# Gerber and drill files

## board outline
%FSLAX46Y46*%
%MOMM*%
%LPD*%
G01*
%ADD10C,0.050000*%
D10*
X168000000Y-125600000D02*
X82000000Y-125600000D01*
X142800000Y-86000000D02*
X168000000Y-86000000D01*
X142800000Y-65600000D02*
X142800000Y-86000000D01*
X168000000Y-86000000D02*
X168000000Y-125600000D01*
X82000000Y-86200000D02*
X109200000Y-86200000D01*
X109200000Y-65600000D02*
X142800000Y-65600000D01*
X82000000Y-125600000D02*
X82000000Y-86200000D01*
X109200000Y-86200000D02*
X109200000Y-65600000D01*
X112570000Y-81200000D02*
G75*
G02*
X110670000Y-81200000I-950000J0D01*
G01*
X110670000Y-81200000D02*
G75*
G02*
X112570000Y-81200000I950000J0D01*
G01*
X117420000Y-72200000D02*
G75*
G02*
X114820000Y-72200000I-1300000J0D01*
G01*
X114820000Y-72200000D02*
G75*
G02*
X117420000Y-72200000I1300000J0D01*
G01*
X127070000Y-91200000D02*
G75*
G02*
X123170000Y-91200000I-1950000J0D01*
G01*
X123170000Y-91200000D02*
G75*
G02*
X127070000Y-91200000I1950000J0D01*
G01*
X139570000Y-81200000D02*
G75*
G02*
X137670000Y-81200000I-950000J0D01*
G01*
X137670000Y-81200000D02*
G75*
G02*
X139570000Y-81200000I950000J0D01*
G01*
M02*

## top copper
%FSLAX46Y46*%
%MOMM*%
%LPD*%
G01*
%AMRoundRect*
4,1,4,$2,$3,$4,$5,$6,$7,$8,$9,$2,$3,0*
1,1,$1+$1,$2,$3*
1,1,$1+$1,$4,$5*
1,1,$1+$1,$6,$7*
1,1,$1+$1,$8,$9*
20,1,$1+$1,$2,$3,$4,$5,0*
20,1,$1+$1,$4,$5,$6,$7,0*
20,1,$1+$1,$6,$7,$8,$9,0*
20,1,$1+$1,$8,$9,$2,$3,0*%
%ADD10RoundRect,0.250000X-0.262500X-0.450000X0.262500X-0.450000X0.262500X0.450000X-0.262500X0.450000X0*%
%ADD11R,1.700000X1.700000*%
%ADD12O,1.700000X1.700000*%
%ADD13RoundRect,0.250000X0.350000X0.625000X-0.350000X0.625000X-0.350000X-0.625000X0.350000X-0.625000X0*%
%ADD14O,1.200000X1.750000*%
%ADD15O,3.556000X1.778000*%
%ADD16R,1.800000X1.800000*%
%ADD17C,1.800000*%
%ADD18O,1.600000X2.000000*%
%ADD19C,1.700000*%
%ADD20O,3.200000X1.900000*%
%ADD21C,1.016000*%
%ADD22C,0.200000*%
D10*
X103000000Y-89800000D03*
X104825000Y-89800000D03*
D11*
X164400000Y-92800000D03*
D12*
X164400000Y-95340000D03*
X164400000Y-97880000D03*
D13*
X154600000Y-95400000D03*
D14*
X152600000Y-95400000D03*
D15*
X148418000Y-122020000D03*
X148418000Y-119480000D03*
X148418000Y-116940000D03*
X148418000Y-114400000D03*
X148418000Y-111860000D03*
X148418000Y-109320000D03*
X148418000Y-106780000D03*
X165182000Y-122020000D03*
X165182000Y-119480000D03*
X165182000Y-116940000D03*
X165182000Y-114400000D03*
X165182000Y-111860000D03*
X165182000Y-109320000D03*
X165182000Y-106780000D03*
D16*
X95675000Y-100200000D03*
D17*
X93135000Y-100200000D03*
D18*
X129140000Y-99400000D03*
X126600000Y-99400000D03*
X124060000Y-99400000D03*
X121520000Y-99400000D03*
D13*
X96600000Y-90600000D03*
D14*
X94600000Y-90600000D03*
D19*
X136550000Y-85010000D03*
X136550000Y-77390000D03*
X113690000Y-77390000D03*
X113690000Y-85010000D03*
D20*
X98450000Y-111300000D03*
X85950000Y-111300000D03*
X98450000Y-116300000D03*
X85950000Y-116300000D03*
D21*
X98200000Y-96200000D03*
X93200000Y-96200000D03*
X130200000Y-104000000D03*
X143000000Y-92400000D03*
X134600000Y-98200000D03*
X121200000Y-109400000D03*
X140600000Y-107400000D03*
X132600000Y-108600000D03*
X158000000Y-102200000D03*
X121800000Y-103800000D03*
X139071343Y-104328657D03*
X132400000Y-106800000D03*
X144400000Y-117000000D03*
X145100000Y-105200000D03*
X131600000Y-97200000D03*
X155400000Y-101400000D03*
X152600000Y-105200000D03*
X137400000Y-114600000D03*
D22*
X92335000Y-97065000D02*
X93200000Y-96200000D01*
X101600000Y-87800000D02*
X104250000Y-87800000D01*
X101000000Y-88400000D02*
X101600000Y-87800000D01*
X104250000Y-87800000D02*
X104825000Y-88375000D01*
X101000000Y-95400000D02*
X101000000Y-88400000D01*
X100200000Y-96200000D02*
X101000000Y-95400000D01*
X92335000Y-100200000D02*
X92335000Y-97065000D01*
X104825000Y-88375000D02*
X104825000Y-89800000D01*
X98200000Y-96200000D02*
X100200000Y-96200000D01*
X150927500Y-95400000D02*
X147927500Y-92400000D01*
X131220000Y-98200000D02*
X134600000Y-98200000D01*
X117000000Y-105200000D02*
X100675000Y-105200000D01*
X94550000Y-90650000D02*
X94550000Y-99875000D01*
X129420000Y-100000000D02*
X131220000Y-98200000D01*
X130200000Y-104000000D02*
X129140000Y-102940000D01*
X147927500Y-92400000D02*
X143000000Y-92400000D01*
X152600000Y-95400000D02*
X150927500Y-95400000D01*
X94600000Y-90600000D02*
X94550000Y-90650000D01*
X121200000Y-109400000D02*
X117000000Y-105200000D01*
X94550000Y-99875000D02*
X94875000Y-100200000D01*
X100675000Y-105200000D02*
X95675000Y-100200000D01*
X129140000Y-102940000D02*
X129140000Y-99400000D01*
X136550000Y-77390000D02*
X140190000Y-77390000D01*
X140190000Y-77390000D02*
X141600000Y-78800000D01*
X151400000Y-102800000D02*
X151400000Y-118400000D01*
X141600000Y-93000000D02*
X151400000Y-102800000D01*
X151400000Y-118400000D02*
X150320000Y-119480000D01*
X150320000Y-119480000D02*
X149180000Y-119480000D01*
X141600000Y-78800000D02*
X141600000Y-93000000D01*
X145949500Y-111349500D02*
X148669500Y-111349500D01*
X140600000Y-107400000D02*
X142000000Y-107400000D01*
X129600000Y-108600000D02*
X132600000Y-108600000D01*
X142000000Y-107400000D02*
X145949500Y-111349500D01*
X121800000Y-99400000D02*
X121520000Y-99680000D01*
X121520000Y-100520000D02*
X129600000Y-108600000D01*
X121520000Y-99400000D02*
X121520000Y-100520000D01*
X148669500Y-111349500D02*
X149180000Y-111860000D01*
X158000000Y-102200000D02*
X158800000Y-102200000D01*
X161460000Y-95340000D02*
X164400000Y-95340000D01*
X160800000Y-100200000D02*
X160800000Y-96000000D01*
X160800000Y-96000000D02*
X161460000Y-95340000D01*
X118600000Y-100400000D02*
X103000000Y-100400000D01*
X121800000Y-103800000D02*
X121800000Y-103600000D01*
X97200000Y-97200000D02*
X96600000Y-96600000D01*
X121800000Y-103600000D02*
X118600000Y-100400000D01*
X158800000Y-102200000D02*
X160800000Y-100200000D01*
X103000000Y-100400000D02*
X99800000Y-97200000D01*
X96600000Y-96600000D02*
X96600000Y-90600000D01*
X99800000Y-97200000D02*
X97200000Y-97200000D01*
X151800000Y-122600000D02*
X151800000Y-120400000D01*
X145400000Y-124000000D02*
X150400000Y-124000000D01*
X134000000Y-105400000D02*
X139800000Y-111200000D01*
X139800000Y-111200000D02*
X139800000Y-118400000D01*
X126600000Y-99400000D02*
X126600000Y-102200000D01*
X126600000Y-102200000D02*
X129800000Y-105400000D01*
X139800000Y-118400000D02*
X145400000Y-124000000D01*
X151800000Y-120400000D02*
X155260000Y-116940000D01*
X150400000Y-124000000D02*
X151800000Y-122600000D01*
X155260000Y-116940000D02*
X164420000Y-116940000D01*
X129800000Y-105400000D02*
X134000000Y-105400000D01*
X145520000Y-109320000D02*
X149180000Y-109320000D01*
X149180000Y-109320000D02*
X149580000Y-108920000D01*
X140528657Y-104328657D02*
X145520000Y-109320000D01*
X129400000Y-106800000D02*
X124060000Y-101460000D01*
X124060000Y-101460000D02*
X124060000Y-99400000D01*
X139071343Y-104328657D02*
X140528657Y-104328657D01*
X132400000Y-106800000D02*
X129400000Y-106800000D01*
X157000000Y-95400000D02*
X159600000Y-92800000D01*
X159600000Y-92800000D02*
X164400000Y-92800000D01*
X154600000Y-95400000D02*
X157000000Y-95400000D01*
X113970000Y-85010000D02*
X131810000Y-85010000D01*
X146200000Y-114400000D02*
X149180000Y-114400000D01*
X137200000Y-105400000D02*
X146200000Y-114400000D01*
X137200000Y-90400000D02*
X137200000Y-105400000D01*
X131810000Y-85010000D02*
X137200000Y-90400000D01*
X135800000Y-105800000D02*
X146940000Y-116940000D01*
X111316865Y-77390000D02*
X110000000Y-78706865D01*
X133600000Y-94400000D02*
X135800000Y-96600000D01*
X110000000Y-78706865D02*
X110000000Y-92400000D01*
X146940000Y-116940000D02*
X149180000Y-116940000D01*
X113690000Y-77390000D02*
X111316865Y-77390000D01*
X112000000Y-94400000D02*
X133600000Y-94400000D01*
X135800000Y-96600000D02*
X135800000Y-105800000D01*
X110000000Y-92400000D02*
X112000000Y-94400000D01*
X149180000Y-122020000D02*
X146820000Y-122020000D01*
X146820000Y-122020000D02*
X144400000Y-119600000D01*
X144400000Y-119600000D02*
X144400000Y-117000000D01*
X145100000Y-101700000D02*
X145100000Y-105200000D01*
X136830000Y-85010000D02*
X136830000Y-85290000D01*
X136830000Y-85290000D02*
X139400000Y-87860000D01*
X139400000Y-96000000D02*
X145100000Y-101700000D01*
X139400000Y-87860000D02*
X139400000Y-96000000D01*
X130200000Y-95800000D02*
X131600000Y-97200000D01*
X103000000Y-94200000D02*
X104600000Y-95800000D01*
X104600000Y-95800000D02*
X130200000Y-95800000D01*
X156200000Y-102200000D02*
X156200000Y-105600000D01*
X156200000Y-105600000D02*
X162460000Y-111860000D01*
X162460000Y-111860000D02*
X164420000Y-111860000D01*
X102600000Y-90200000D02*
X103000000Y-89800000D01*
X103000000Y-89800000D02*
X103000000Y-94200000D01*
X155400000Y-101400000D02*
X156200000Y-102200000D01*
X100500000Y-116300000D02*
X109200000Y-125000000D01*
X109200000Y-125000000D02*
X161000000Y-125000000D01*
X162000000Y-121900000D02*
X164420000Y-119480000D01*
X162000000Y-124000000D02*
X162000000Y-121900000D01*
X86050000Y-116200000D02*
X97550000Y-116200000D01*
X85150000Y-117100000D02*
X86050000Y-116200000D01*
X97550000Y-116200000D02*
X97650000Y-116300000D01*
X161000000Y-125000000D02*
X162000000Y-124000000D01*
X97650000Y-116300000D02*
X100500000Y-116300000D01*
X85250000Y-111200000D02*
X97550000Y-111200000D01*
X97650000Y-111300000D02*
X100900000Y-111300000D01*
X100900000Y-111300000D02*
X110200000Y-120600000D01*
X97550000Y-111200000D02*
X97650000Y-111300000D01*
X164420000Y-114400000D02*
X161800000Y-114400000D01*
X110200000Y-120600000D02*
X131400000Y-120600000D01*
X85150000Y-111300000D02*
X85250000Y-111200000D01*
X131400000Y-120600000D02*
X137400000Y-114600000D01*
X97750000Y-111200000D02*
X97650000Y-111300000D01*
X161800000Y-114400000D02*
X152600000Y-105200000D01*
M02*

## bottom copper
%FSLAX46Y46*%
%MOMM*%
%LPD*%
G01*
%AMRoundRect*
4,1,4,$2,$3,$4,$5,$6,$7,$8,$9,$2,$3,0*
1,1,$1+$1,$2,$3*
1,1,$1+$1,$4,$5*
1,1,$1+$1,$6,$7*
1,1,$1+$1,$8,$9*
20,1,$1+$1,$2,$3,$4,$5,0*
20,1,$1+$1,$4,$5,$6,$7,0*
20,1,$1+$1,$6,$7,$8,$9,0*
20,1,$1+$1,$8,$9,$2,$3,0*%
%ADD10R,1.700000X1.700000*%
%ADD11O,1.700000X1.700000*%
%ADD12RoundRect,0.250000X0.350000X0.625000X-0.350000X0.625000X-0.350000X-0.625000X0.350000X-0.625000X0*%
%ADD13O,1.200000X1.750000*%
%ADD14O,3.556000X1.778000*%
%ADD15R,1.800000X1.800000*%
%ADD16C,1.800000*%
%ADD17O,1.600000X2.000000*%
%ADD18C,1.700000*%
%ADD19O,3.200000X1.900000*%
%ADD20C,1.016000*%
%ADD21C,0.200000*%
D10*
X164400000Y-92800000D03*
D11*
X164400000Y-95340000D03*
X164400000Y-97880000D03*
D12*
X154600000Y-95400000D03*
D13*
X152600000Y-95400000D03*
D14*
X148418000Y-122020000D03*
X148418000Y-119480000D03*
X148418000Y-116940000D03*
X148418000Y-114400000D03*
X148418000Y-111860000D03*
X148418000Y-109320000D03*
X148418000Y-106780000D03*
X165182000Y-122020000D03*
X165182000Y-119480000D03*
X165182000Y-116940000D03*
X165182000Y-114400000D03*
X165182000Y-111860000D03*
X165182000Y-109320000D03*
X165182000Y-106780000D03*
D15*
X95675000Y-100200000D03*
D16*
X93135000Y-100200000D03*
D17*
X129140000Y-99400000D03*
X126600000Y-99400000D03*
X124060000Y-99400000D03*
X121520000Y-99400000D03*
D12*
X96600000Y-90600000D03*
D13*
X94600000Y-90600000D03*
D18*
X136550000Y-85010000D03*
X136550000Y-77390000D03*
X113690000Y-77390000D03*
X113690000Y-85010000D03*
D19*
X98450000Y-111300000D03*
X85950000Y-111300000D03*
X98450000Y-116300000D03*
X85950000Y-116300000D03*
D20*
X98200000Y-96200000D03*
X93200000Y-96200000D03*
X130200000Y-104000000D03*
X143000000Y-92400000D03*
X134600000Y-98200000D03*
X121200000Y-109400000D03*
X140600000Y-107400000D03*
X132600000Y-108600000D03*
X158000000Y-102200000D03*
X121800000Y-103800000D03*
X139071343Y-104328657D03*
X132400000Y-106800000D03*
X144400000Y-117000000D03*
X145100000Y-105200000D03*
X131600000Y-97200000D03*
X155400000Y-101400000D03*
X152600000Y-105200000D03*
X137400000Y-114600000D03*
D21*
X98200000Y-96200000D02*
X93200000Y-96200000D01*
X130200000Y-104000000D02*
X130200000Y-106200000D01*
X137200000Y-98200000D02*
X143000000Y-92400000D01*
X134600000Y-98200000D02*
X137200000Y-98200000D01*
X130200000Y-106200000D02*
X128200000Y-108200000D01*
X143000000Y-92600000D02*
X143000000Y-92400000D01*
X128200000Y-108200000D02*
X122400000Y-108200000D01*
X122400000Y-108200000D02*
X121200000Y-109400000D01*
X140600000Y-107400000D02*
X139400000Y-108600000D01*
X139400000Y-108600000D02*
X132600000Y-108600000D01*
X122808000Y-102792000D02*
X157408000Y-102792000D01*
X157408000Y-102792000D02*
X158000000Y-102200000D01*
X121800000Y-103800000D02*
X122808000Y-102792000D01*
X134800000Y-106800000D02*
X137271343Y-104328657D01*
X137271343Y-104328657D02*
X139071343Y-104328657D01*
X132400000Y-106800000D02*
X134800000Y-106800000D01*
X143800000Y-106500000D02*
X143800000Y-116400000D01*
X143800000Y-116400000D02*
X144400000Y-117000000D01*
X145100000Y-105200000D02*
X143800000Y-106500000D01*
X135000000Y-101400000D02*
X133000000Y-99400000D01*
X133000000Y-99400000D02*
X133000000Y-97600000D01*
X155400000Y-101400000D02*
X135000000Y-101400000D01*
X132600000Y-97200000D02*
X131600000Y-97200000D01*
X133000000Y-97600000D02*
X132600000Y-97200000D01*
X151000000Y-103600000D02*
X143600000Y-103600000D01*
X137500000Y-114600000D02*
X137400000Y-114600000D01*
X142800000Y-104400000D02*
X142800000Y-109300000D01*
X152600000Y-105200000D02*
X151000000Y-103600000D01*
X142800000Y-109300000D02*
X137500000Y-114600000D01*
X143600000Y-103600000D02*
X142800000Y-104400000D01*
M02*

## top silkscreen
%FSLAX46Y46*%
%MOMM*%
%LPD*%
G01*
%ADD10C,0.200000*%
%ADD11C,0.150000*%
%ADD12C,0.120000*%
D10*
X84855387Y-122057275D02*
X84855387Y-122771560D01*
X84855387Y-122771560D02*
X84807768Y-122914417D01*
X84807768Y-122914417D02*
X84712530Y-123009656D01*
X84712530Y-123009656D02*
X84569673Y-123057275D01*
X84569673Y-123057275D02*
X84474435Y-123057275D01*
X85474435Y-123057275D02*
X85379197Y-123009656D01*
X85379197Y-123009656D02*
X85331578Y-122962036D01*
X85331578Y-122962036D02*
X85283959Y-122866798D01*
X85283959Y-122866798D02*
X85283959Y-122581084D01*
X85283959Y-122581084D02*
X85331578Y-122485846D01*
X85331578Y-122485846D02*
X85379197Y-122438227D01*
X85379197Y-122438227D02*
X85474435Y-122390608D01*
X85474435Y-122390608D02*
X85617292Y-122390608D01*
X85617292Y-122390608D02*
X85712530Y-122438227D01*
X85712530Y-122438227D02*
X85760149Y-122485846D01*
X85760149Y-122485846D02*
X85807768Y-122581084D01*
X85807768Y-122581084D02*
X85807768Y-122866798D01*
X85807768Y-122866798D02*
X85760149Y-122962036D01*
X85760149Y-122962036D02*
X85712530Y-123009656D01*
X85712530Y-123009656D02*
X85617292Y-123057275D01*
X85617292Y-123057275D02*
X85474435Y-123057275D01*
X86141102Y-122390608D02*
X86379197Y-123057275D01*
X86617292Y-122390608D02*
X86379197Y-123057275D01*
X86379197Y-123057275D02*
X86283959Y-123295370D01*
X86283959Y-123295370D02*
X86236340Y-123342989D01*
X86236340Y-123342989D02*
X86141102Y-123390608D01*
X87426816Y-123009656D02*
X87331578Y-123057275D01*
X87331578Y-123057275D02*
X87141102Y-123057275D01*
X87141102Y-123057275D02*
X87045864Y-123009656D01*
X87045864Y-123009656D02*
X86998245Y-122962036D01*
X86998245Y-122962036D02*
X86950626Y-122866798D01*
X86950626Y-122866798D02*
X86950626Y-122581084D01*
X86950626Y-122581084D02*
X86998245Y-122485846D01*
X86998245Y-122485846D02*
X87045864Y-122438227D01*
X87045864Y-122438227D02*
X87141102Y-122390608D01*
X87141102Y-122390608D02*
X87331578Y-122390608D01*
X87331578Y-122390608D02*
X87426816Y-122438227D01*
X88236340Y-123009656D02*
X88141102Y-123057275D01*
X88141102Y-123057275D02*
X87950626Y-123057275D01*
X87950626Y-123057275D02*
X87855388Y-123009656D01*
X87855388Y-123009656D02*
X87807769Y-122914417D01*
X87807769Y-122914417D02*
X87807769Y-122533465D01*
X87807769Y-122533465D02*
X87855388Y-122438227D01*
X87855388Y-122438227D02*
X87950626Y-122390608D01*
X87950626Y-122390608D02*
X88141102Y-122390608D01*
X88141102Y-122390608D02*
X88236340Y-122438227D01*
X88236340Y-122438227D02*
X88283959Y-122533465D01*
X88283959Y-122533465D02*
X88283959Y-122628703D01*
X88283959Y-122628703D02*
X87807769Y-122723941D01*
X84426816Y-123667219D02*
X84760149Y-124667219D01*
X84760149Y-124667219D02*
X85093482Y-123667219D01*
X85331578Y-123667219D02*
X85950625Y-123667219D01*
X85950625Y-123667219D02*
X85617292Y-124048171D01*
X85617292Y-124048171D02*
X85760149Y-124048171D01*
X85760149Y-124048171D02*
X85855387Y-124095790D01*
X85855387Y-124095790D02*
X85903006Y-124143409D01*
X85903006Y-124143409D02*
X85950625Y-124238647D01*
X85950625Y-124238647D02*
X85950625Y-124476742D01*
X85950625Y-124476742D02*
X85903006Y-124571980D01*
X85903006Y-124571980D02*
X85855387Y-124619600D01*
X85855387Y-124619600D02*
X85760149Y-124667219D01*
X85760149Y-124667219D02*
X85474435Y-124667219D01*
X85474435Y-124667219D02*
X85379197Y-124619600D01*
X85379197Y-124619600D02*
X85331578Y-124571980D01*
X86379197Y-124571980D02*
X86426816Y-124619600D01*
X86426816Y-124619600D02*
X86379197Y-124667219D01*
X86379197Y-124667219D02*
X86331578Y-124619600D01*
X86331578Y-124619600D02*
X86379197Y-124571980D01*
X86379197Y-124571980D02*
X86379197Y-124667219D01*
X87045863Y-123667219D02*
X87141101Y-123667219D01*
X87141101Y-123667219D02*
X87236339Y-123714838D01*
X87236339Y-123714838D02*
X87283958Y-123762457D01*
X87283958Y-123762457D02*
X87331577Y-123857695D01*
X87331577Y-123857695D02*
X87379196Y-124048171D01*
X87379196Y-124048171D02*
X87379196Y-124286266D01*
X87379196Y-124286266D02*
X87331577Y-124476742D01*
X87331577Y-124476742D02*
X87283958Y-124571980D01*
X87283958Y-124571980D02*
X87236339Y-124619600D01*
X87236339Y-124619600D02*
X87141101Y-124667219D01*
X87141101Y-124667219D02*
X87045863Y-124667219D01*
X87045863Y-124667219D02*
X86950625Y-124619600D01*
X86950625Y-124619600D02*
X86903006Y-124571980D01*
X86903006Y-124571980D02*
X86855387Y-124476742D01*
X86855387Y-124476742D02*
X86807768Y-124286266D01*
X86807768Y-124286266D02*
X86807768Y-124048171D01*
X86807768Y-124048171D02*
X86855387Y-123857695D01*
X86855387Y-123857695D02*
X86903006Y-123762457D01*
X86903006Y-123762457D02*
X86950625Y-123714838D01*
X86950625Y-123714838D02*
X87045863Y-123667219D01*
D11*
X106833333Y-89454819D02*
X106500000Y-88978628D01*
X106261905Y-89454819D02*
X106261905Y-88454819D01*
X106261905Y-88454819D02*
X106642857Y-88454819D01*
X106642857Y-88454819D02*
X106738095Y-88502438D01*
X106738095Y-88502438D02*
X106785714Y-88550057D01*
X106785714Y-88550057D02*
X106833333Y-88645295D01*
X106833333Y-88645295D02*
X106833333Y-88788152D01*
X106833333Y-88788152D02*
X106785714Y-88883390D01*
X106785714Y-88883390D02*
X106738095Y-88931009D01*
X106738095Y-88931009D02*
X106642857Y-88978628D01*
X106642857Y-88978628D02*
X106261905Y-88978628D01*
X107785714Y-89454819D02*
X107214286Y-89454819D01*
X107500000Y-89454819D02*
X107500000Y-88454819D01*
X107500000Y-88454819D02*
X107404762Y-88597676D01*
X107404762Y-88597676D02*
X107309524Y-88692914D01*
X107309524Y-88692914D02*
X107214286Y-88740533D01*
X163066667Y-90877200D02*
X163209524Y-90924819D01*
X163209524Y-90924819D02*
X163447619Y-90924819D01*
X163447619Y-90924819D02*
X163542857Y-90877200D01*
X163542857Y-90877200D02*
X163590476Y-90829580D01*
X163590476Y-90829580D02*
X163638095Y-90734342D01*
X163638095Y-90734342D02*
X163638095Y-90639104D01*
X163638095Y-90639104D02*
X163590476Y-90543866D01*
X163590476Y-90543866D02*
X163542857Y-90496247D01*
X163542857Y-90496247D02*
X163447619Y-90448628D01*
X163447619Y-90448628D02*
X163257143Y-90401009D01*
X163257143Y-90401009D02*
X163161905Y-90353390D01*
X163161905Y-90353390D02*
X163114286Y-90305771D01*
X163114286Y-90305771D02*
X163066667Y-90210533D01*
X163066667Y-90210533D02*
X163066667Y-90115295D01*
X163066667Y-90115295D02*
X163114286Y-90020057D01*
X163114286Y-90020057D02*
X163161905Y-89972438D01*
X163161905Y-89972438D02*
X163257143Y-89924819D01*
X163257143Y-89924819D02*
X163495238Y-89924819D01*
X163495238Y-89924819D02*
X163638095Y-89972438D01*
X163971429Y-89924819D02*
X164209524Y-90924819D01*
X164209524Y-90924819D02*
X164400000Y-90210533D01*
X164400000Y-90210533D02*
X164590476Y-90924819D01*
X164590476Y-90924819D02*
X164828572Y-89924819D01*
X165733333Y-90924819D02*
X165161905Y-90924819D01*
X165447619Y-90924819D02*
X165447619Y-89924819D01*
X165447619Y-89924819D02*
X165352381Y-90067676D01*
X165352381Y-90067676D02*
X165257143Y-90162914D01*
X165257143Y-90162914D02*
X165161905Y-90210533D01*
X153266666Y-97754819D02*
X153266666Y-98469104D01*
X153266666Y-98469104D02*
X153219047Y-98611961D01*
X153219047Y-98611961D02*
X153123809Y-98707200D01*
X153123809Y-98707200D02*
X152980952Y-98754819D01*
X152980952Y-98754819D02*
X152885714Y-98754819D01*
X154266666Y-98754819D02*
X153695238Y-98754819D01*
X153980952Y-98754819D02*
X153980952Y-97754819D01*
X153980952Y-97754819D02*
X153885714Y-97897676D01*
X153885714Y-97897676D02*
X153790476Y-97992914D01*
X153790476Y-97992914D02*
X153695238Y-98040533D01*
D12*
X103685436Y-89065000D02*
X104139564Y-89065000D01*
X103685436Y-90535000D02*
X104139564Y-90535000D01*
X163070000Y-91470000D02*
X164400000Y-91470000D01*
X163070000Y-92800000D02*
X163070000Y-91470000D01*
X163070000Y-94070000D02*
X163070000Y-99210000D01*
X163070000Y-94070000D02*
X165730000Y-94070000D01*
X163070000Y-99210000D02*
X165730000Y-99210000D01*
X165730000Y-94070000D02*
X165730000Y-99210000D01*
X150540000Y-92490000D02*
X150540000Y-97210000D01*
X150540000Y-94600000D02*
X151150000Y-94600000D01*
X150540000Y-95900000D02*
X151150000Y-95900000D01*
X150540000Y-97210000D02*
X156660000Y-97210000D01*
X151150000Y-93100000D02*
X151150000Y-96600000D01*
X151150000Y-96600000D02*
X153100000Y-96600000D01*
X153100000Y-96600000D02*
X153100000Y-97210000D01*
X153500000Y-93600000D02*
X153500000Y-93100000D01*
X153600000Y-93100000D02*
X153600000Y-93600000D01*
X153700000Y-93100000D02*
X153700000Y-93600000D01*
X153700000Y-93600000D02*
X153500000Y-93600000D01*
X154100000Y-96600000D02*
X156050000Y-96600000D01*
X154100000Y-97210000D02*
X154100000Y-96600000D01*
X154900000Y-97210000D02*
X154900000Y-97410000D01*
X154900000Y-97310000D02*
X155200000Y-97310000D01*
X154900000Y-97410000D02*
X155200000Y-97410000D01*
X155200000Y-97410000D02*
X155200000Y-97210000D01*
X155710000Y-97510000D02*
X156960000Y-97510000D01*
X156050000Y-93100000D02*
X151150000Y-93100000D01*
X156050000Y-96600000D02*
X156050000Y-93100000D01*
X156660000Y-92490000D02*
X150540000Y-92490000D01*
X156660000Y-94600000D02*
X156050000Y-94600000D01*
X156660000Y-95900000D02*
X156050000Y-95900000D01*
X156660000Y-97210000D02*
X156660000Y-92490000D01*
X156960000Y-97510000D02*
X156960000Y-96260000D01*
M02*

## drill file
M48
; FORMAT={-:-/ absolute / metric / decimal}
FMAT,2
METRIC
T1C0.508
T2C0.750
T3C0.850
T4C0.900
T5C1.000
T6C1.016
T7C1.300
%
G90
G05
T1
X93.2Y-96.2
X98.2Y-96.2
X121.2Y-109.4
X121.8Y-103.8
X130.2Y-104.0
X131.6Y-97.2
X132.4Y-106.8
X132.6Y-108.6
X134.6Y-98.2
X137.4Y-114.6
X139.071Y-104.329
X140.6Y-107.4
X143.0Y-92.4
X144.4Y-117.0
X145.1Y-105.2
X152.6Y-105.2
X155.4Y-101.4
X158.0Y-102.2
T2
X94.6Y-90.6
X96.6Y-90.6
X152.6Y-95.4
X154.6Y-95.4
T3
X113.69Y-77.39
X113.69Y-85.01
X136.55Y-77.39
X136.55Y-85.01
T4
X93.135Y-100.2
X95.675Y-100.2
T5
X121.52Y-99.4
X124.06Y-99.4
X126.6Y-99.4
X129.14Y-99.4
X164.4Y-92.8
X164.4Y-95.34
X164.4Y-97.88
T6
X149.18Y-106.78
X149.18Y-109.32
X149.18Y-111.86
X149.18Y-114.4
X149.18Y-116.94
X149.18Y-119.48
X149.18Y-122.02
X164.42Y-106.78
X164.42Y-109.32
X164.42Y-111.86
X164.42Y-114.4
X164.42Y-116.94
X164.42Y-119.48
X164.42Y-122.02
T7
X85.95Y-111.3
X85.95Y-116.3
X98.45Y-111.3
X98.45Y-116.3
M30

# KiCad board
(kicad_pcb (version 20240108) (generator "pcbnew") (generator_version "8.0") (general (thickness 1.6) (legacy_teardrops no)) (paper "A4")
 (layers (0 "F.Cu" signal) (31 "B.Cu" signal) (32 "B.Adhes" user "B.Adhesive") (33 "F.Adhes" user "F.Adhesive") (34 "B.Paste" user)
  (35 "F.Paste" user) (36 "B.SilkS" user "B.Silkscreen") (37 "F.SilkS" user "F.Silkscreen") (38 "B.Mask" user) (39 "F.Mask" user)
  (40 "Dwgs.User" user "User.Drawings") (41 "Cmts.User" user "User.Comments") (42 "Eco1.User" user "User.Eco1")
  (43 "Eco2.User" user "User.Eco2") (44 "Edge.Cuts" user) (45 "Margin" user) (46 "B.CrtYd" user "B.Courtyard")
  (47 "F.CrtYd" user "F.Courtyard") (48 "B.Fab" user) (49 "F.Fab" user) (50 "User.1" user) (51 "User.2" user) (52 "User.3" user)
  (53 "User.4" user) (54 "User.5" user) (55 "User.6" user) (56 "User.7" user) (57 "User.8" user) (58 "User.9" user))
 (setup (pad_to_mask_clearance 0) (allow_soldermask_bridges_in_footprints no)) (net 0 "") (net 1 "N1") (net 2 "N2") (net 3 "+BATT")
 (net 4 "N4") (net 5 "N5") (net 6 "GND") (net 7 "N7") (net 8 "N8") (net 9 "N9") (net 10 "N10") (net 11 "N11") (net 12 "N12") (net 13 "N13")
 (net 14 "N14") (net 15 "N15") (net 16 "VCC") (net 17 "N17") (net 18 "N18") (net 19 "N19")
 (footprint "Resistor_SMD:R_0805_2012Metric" (layer "F.Cu") (at 103.9125 89.8)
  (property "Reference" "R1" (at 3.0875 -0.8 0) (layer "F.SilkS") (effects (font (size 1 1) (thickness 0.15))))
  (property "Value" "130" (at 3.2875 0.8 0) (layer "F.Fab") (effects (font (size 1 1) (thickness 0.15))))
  (fp_line (start -0.227064 -0.735) (end 0.227064 -0.735) (stroke (width 0.12) (type solid)) (layer "F.SilkS"))
  (fp_line (start -0.227064 0.735) (end 0.227064 0.735) (stroke (width 0.12) (type solid)) (layer "F.SilkS"))
  (pad "1" smd roundrect (at -0.9125 0) (size 1.025 1.4) (layers "F.Cu" "F.Paste" "F.Mask") (roundrect_rratio 0.243902) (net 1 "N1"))
  (pad "2" smd roundrect (at 0.9125 0) (size 1.025 1.4) (layers "F.Cu" "F.Paste" "F.Mask") (roundrect_rratio 0.243902) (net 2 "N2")))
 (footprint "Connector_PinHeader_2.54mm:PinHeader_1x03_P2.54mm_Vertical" (layer "F.Cu") (at 164.4 92.8)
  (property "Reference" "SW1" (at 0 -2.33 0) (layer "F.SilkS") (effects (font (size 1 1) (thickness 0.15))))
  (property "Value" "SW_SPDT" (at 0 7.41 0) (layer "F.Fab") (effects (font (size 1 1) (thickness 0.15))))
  (fp_line (start -1.33 -1.33) (end 0 -1.33) (stroke (width 0.12) (type solid)) (layer "F.SilkS"))
  (fp_line (start -1.33 0) (end -1.33 -1.33) (stroke (width 0.12) (type solid)) (layer "F.SilkS"))
  (fp_line (start -1.33 1.27) (end -1.33 6.41) (stroke (width 0.12) (type solid)) (layer "F.SilkS"))
  (fp_line (start -1.33 1.27) (end 1.33 1.27) (stroke (width 0.12) (type solid)) (layer "F.SilkS"))
  (fp_line (start -1.33 6.41) (end 1.33 6.41) (stroke (width 0.12) (type solid)) (layer "F.SilkS"))
  (fp_line (start 1.33 1.27) (end 1.33 6.41) (stroke (width 0.12) (type solid)) (layer "F.SilkS"))
  (pad "1" thru_hole rect (at 0 0) (size 1.7 1.7) (drill 1) (layers "*.Cu" "*.Mask") (remove_unused_layers no) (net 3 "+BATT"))
  (pad "2" thru_hole oval (at 0 2.54) (size 1.7 1.7) (drill 1) (layers "*.Cu" "*.Mask") (remove_unused_layers no) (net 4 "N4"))
  (pad "3" thru_hole oval (at 0 5.08) (size 1.7 1.7) (drill 1) (layers "*.Cu" "*.Mask") (remove_unused_layers no) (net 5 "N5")))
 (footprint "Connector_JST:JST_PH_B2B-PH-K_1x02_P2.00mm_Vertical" (layer "F.Cu") (at 154.6 95.4 180)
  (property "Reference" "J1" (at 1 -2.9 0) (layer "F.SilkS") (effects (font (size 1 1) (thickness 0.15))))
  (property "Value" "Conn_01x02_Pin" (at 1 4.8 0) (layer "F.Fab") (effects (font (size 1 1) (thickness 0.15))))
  (fp_line (start 4.06 2.91) (end 4.06 -1.81) (stroke (width 0.12) (type solid)) (layer "F.SilkS"))
  (fp_line (start 4.06 0.8) (end 3.45 0.8) (stroke (width 0.12) (type solid)) (layer "F.SilkS"))
  (fp_line (start 4.06 -0.5) (end 3.45 -0.5) (stroke (width 0.12) (type solid)) (layer "F.SilkS"))
  (fp_line (start 4.06 -1.81) (end -2.06 -1.81) (stroke (width 0.12) (type solid)) (layer "F.SilkS"))
  (fp_line (start 3.45 2.3) (end 3.45 -1.2) (stroke (width 0.12) (type solid)) (layer "F.SilkS"))
  (fp_line (start 3.45 -1.2) (end 1.5 -1.2) (stroke (width 0.12) (type solid)) (layer "F.SilkS"))
  (fp_line (start 1.5 -1.2) (end 1.5 -1.81) (stroke (width 0.12) (type solid)) (layer "F.SilkS"))
  (fp_line (start 1.1 1.8) (end 1.1 2.3) (stroke (width 0.12) (type solid)) (layer "F.SilkS"))
  (fp_line (start 1 2.3) (end 1 1.8) (stroke (width 0.12) (type solid)) (layer "F.SilkS"))
  (fp_line (start 0.9 2.3) (end 0.9 1.8) (stroke (width 0.12) (type solid)) (layer "F.SilkS"))
  (fp_line (start 0.9 1.8) (end 1.1 1.8) (stroke (width 0.12) (type solid)) (layer "F.SilkS"))
  (fp_line (start 0.5 -1.2) (end -1.45 -1.2) (stroke (width 0.12) (type solid)) (layer "F.SilkS"))
  (fp_line (start 0.5 -1.81) (end 0.5 -1.2) (stroke (width 0.12) (type solid)) (layer "F.SilkS"))
  (fp_line (start -0.3 -1.81) (end -0.3 -2.01) (stroke (width 0.12) (type solid)) (layer "F.SilkS"))
  (fp_line (start -0.3 -1.91) (end -0.6 -1.91) (stroke (width 0.12) (type solid)) (layer "F.SilkS"))
  (fp_line (start -0.3 -2.01) (end -0.6 -2.01) (stroke (width 0.12) (type solid)) (layer "F.SilkS"))
  (fp_line (start -0.6 -2.01) (end -0.6 -1.81) (stroke (width 0.12) (type solid)) (layer "F.SilkS"))
  (fp_line (start -1.11 -2.11) (end -2.36 -2.11) (stroke (width 0.12) (type solid)) (layer "F.SilkS"))
  (fp_line (start -1.45 2.3) (end 3.45 2.3) (stroke (width 0.12) (type solid)) (layer "F.SilkS"))
  (fp_line (start -1.45 -1.2) (end -1.45 2.3) (stroke (width 0.12) (type solid)) (layer "F.SilkS"))
  (fp_line (start -2.06 2.91) (end 4.06 2.91) (stroke (width 0.12) (type solid)) (layer "F.SilkS"))
  (fp_line (start -2.06 0.8) (end -1.45 0.8) (stroke (width 0.12) (type solid)) (layer "F.SilkS"))
  (fp_line (start -2.06 -0.5) (end -1.45 -0.5) (stroke (width 0.12) (type solid)) (layer "F.SilkS"))
  (fp_line (start -2.06 -1.81) (end -2.06 2.91) (stroke (width 0.12) (type solid)) (layer "F.SilkS"))
  (fp_line (start -2.36 -2.11) (end -2.36 -0.86) (stroke (width 0.12) (type solid)) (layer "F.SilkS"))
  (pad "1" thru_hole roundrect (at 0 0 180) (size 1.2 1.75) (drill 0.75) (layers "*.Cu" "*.Mask") (remove_unused_layers no)
   (roundrect_rratio 0.208333) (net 3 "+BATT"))
  (pad "2" thru_hole oval (at 2 0 180) (size 1.2 1.75) (drill 0.75) (layers "*.Cu" "*.Mask") (remove_unused_layers no) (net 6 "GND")))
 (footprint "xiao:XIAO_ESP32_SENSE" (layer "B.Cu") (at 156.8 114.4)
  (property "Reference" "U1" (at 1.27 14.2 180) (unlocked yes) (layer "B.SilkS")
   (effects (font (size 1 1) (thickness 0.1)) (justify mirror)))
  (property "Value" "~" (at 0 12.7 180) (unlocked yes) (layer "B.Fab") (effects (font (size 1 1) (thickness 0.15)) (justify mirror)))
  (pad "1" thru_hole oval (at -7.62 7.62) (size 3.556 1.778) (drill 1.016 (offset -0.762 0)) (layers "*.Cu" "*.Mask")
   (remove_unused_layers no) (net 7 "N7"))
  (pad "2" thru_hole oval (at -7.62 5.08) (size 3.556 1.778) (drill 1.016 (offset -0.762 0)) (layers "*.Cu" "*.Mask")
   (remove_unused_layers no) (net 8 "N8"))
  (pad "3" thru_hole oval (at -7.62 2.54) (size 3.556 1.778) (drill 1.016 (offset -0.762 0)) (layers "*.Cu" "*.Mask")
   (remove_unused_layers no) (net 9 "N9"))
  (pad "4" thru_hole oval (at -7.62 0) (size 3.556 1.778) (drill 1.016 (offset -0.762 0)) (layers "*.Cu" "*.Mask") (remove_unused_layers no)
   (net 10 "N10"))
  (pad "5" thru_hole oval (at -7.62 -2.54) (size 3.556 1.778) (drill 1.016 (offset -0.762 0)) (layers "*.Cu" "*.Mask")
   (remove_unused_layers no) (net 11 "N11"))
  (pad "6" thru_hole oval (at -7.62 -5.08) (size 3.556 1.778) (drill 1.016 (offset -0.762 0)) (layers "*.Cu" "*.Mask")
   (remove_unused_layers no) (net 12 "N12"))
  (pad "7" thru_hole oval (at -7.62 -7.62) (size 3.556 1.778) (drill 1.016 (offset -0.762 0)) (layers "*.Cu" "*.Mask")
   (remove_unused_layers no) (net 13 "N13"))
  (pad "8" thru_hole oval (at 7.62 7.62) (size 3.556 1.778) (drill 1.016 (offset 0.762 0)) (layers "*.Cu" "*.Mask")
   (remove_unused_layers no) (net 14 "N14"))
  (pad "9" thru_hole oval (at 7.62 5.08) (size 3.556 1.778) (drill 1.016 (offset 0.762 0)) (layers "*.Cu" "*.Mask")
   (remove_unused_layers no) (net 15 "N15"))
  (pad "10" thru_hole oval (at 7.62 2.54) (size 3.556 1.778) (drill 1.016 (offset 0.762 0)) (layers "*.Cu" "*.Mask")
   (remove_unused_layers no) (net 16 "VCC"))
  (pad "11" thru_hole oval (at 7.62 0) (size 3.556 1.778) (drill 1.016 (offset 0.762 0)) (layers "*.Cu" "*.Mask") (remove_unused_layers no)
   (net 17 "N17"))
  (pad "12" thru_hole oval (at 7.62 -2.54) (size 3.556 1.778) (drill 1.016 (offset 0.762 0)) (layers "*.Cu" "*.Mask")
   (remove_unused_layers no) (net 1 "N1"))
  (pad "13" thru_hole oval (at 7.62 -5.08) (size 3.556 1.778) (drill 1.016 (offset 0.762 0)) (layers "*.Cu" "*.Mask")
   (remove_unused_layers no) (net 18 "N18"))
  (pad "14" thru_hole oval (at 7.62 -7.62) (size 3.556 1.778) (drill 1.016 (offset 0.762 0)) (layers "*.Cu" "*.Mask")
   (remove_unused_layers no) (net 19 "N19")))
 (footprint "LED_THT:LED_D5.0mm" (layer "B.Cu") (at 95.675 100.2 180)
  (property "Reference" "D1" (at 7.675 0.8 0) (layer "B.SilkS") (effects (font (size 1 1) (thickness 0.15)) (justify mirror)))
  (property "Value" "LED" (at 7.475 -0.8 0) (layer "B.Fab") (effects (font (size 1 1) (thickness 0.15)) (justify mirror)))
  (pad "1" thru_hole rect (at 0 0 180) (size 1.8 1.8) (drill 0.9) (layers "*.Cu" "*.Mask") (remove_unused_layers no) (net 6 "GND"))
  (pad "2" thru_hole circle (at 2.54 0 180) (size 1.8 1.8) (drill 0.9) (layers "*.Cu" "*.Mask") (remove_unused_layers no) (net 2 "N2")))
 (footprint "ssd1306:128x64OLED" (layer "B.Cu") (at 125.52 110 180)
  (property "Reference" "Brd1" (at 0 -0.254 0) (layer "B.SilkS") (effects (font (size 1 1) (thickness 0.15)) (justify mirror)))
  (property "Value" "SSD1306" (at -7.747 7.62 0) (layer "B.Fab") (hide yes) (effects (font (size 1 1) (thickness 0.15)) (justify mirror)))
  (pad "1" thru_hole oval (at -3.62 10.6 90) (size 2 1.6) (drill 1) (layers "*.Cu" "*.Mask") (remove_unused_layers no) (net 6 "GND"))
  (pad "2" thru_hole oval (at -1.08 10.6 90) (size 2 1.6) (drill 1) (layers "*.Cu" "*.Mask") (remove_unused_layers no) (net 16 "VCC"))
  (pad "3" thru_hole oval (at 1.46 10.6 90) (size 2 1.6) (drill 1) (layers "*.Cu" "*.Mask") (remove_unused_layers no) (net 12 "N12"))
  (pad "4" thru_hole oval (at 4 10.6 90) (size 2 1.6) (drill 1) (layers "*.Cu" "*.Mask") (remove_unused_layers no) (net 11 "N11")))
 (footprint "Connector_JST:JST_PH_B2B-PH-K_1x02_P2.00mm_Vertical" (layer "B.Cu") (at 96.6 90.6 180)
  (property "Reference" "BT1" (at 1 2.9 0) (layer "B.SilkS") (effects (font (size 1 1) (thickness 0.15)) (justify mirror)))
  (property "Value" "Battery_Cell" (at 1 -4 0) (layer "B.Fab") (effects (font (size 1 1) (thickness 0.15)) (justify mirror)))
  (pad "1" thru_hole roundrect (at 0 0 180) (size 1.2 1.75) (drill 0.75) (layers "*.Cu" "*.Mask") (remove_unused_layers no)
   (roundrect_rratio 0.208333) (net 4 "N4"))
  (pad "2" thru_hole oval (at 2 0 180) (size 1.2 1.75) (drill 0.75) (layers "*.Cu" "*.Mask") (remove_unused_layers no) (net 6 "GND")))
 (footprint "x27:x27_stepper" (layer "B.Cu") (at 127.66 71.04)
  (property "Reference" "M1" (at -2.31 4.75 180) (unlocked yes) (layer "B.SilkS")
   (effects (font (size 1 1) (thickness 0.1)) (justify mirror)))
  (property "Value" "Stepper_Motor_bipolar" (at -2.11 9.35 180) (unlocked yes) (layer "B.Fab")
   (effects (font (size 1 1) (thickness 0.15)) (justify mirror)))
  (fp_circle (center -16.04 10.16) (end -15.09 10.16) (stroke (width 0.05) (type default)) (fill none) (layer "Edge.Cuts"))
  (fp_circle (center -11.54 1.16) (end -10.24 1.16) (stroke (width 0.05) (type default)) (fill none) (layer "Edge.Cuts"))
  (fp_circle (center -2.54 20.16) (end -0.59 20.16) (stroke (width 0.05) (type default)) (fill none) (layer "Edge.Cuts"))
  (fp_circle (center 10.96 10.16) (end 11.91 10.16) (stroke (width 0.05) (type default)) (fill none) (layer "Edge.Cuts"))
  (pad "1" thru_hole circle (at 8.89 13.97) (size 1.7 1.7) (drill 0.85) (layers "*.Cu" "*.Mask") (remove_unused_layers no) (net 7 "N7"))
  (pad "2" thru_hole circle (at 8.89 6.35) (size 1.7 1.7) (drill 0.85) (layers "*.Cu" "*.Mask") (remove_unused_layers no) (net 8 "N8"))
  (pad "3" thru_hole circle (at -13.97 6.35) (size 1.7 1.7) (drill 0.85) (layers "*.Cu" "*.Mask") (remove_unused_layers no) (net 9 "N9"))
  (pad "4" thru_hole circle (at -13.97 13.97) (size 1.7 1.7) (drill 0.85) (layers "*.Cu" "*.Mask") (remove_unused_layers no) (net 10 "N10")))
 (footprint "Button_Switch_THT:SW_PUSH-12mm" (layer "B.Cu") (at 98.45 111.3 180)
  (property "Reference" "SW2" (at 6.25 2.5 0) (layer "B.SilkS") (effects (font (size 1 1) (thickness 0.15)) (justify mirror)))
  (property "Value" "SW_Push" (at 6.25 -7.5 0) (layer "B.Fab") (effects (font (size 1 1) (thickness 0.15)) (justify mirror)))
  (pad "1" thru_hole oval (at 0 0 180) (size 3.2 1.9) (drill 1.3) (layers "*.Cu" "*.Mask") (remove_unused_layers no) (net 17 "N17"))
  (pad "1" thru_hole oval (at 12.5 0 180) (size 3.2 1.9) (drill 1.3) (layers "*.Cu" "*.Mask") (remove_unused_layers no) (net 17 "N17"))
  (pad "2" thru_hole oval (at 0 -5 180) (size 3.2 1.9) (drill 1.3) (layers "*.Cu" "*.Mask") (remove_unused_layers no) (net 15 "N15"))
  (pad "2" thru_hole oval (at 12.5 -5 180) (size 3.2 1.9) (drill 1.3) (layers "*.Cu" "*.Mask") (remove_unused_layers no) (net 15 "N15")))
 (gr_line (start 168 125.6) (end 82 125.6) (stroke (width 0.05) (type default)) (layer "Edge.Cuts"))
 (gr_line (start 142.8 86) (end 168 86) (stroke (width 0.05) (type default)) (layer "Edge.Cuts"))
 (gr_line (start 142.8 65.6) (end 142.8 86) (stroke (width 0.05) (type default)) (layer "Edge.Cuts"))
 (gr_line (start 168 86) (end 168 125.6) (stroke (width 0.05) (type default)) (layer "Edge.Cuts"))
 (gr_line (start 82 86.2) (end 109.2 86.2) (stroke (width 0.05) (type default)) (layer "Edge.Cuts"))
 (gr_line (start 109.2 65.6) (end 142.8 65.6) (stroke (width 0.05) (type default)) (layer "Edge.Cuts"))
 (gr_line (start 82 125.6) (end 82 86.2) (stroke (width 0.05) (type default)) (layer "Edge.Cuts"))
 (gr_line (start 109.2 86.2) (end 109.2 65.6) (stroke (width 0.05) (type default)) (layer "Edge.Cuts"))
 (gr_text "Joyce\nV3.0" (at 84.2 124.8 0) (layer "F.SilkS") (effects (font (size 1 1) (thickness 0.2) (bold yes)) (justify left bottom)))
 (segment (start 92.335 97.065) (end 93.2 96.2) (width 0.2) (layer "F.Cu") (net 2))
 (segment (start 101.6 87.8) (end 104.25 87.8) (width 0.2) (layer "F.Cu") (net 2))
 (segment (start 101 88.4) (end 101.6 87.8) (width 0.2) (layer "F.Cu") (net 2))
 (segment (start 104.25 87.8) (end 104.825 88.375) (width 0.2) (layer "F.Cu") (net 2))
 (segment (start 101 95.4) (end 101 88.4) (width 0.2) (layer "F.Cu") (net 2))
 (segment (start 100.2 96.2) (end 101 95.4) (width 0.2) (layer "F.Cu") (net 2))
 (segment (start 92.335 100.2) (end 92.335 97.065) (width 0.2) (layer "F.Cu") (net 2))
 (segment (start 104.825 88.375) (end 104.825 89.8) (width 0.2) (layer "F.Cu") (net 2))
 (segment (start 98.2 96.2) (end 100.2 96.2) (width 0.2) (layer "F.Cu") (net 2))
 (via (at 98.2 96.2) (size 1.016) (drill 0.508) (layers "F.Cu" "B.Cu") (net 2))
 (via (at 93.2 96.2) (size 1.016) (drill 0.508) (layers "F.Cu" "B.Cu") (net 2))
 (segment (start 98.2 96.2) (end 93.2 96.2) (width 0.2) (layer "B.Cu") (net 2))
 (segment (start 150.9275 95.4) (end 147.9275 92.4) (width 0.2) (layer "F.Cu") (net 6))
 (segment (start 131.22 98.2) (end 134.6 98.2) (width 0.2) (layer "F.Cu") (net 6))
 (segment (start 117 105.2) (end 100.675 105.2) (width 0.2) (layer "F.Cu") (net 6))
 (segment (start 94.55 90.65) (end 94.55 99.875) (width 0.2) (layer "F.Cu") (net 6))
 (segment (start 129.42 100) (end 131.22 98.2) (width 0.2) (layer "F.Cu") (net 6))
 (segment (start 130.2 104) (end 129.14 102.94) (width 0.2) (layer "F.Cu") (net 6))
 (segment (start 147.9275 92.4) (end 143 92.4) (width 0.2) (layer "F.Cu") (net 6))
 (segment (start 152.6 95.4) (end 150.9275 95.4) (width 0.2) (layer "F.Cu") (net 6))
 (segment (start 94.6 90.6) (end 94.55 90.65) (width 0.2) (layer "F.Cu") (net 6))
 (segment (start 121.2 109.4) (end 117 105.2) (width 0.2) (layer "F.Cu") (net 6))
 (segment (start 94.55 99.875) (end 94.875 100.2) (width 0.2) (layer "F.Cu") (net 6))
 (segment (start 100.675 105.2) (end 95.675 100.2) (width 0.2) (layer "F.Cu") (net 6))
 (segment (start 129.14 102.94) (end 129.14 99.4) (width 0.2) (layer "F.Cu") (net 6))
 (via (at 130.2 104) (size 1.016) (drill 0.508) (layers "F.Cu" "B.Cu") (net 6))
 (via (at 143 92.4) (size 1.016) (drill 0.508) (layers "F.Cu" "B.Cu") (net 6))
 (via (at 134.6 98.2) (size 1.016) (drill 0.508) (layers "F.Cu" "B.Cu") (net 6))
 (via (at 121.2 109.4) (size 1.016) (drill 0.508) (layers "F.Cu" "B.Cu") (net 6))
 (segment (start 130.2 104) (end 130.2 106.2) (width 0.2) (layer "B.Cu") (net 6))
 (segment (start 137.2 98.2) (end 143 92.4) (width 0.2) (layer "B.Cu") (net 6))
 (segment (start 134.6 98.2) (end 137.2 98.2) (width 0.2) (layer "B.Cu") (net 6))
 (segment (start 130.2 106.2) (end 128.2 108.2) (width 0.2) (layer "B.Cu") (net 6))
 (segment (start 143 92.6) (end 143 92.4) (width 0.2) (layer "B.Cu") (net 6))
 (segment (start 128.2 108.2) (end 122.4 108.2) (width 0.2) (layer "B.Cu") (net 6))
 (segment (start 122.4 108.2) (end 121.2 109.4) (width 0.2) (layer "B.Cu") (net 6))
 (segment (start 136.55 77.39) (end 140.19 77.39) (width 0.2) (layer "F.Cu") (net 8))
 (segment (start 140.19 77.39) (end 141.6 78.8) (width 0.2) (layer "F.Cu") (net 8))
 (segment (start 151.4 102.8) (end 151.4 118.4) (width 0.2) (layer "F.Cu") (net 8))
 (segment (start 141.6 93) (end 151.4 102.8) (width 0.2) (layer "F.Cu") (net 8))
 (segment (start 151.4 118.4) (end 150.32 119.48) (width 0.2) (layer "F.Cu") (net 8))
 (segment (start 150.32 119.48) (end 149.18 119.48) (width 0.2) (layer "F.Cu") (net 8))
 (segment (start 141.6 78.8) (end 141.6 93) (width 0.2) (layer "F.Cu") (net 8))
 (segment (start 145.9495 111.3495) (end 148.6695 111.3495) (width 0.2) (layer "F.Cu") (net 11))
 (segment (start 140.6 107.4) (end 142 107.4) (width 0.2) (layer "F.Cu") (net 11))
 (segment (start 129.6 108.6) (end 132.6 108.6) (width 0.2) (layer "F.Cu") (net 11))
 (segment (start 142 107.4) (end 145.9495 111.3495) (width 0.2) (layer "F.Cu") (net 11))
 (segment (start 121.8 99.4) (end 121.52 99.68) (width 0.2) (layer "F.Cu") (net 11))
 (segment (start 121.52 100.52) (end 129.6 108.6) (width 0.2) (layer "F.Cu") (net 11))
 (segment (start 121.52 99.4) (end 121.52 100.52) (width 0.2) (layer "F.Cu") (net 11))
 (segment (start 148.6695 111.3495) (end 149.18 111.86) (width 0.2) (layer "F.Cu") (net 11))
 (via (at 140.6 107.4) (size 1.016) (drill 0.508) (layers "F.Cu" "B.Cu") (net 11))
 (via (at 132.6 108.6) (size 1.016) (drill 0.508) (layers "F.Cu" "B.Cu") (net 11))
 (segment (start 140.6 107.4) (end 139.4 108.6) (width 0.2) (layer "B.Cu") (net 11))
 (segment (start 139.4 108.6) (end 132.6 108.6) (width 0.2) (layer "B.Cu") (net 11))
 (segment (start 158 102.2) (end 158.8 102.2) (width 0.2) (layer "F.Cu") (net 4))
 (segment (start 161.46 95.34) (end 164.4 95.34) (width 0.2) (layer "F.Cu") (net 4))
 (segment (start 160.8 100.2) (end 160.8 96) (width 0.2) (layer "F.Cu") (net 4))
 (segment (start 160.8 96) (end 161.46 95.34) (width 0.2) (layer "F.Cu") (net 4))
 (segment (start 118.6 100.4) (end 103 100.4) (width 0.2) (layer "F.Cu") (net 4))
 (segment (start 121.8 103.8) (end 121.8 103.6) (width 0.2) (layer "F.Cu") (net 4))
 (segment (start 97.2 97.2) (end 96.6 96.6) (width 0.2) (layer "F.Cu") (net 4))
 (segment (start 121.8 103.6) (end 118.6 100.4) (width 0.2) (layer "F.Cu") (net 4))
 (segment (start 158.8 102.2) (end 160.8 100.2) (width 0.2) (layer "F.Cu") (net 4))
 (segment (start 103 100.4) (end 99.8 97.2) (width 0.2) (layer "F.Cu") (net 4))
 (segment (start 96.6 96.6) (end 96.6 90.6) (width 0.2) (layer "F.Cu") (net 4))
 (segment (start 99.8 97.2) (end 97.2 97.2) (width 0.2) (layer "F.Cu") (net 4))
 (via (at 158 102.2) (size 1.016) (drill 0.508) (layers "F.Cu" "B.Cu") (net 4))
 (via (at 121.8 103.8) (size 1.016) (drill 0.508) (layers "F.Cu" "B.Cu") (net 4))
 (segment (start 122.808 102.792) (end 157.408 102.792) (width 0.2) (layer "B.Cu") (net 4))
 (segment (start 157.408 102.792) (end 158 102.2) (width 0.2) (layer "B.Cu") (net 4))
 (segment (start 121.8 103.8) (end 122.808 102.792) (width 0.2) (layer "B.Cu") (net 4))
 (segment (start 151.8 122.6) (end 151.8 120.4) (width 0.2) (layer "F.Cu") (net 16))
 (segment (start 145.4 124) (end 150.4 124) (width 0.2) (layer "F.Cu") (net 16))
 (segment (start 134 105.4) (end 139.8 111.2) (width 0.2) (layer "F.Cu") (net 16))
 (segment (start 139.8 111.2) (end 139.8 118.4) (width 0.2) (layer "F.Cu") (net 16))
 (segment (start 126.6 99.4) (end 126.6 102.2) (width 0.2) (layer "F.Cu") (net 16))
 (segment (start 126.6 102.2) (end 129.8 105.4) (width 0.2) (layer "F.Cu") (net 16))
 (segment (start 139.8 118.4) (end 145.4 124) (width 0.2) (layer "F.Cu") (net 16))
 (segment (start 151.8 120.4) (end 155.26 116.94) (width 0.2) (layer "F.Cu") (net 16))
 (segment (start 150.4 124) (end 151.8 122.6) (width 0.2) (layer "F.Cu") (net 16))
 (segment (start 155.26 116.94) (end 164.42 116.94) (width 0.2) (layer "F.Cu") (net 16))
 (segment (start 129.8 105.4) (end 134 105.4) (width 0.2) (layer "F.Cu") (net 16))
 (segment (start 145.52 109.32) (end 149.18 109.32) (width 0.2) (layer "F.Cu") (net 12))
 (segment (start 149.18 109.32) (end 149.58 108.92) (width 0.2) (layer "F.Cu") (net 12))
 (segment (start 140.528657 104.328657) (end 145.52 109.32) (width 0.2) (layer "F.Cu") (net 12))
 (segment (start 129.4 106.8) (end 124.06 101.46) (width 0.2) (layer "F.Cu") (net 12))
 (segment (start 124.06 101.46) (end 124.06 99.4) (width 0.2) (layer "F.Cu") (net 12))
 (segment (start 139.071343 104.328657) (end 140.528657 104.328657) (width 0.2) (layer "F.Cu") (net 12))
 (segment (start 132.4 106.8) (end 129.4 106.8) (width 0.2) (layer "F.Cu") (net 12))
 (via (at 139.071343 104.328657) (size 1.016) (drill 0.508) (layers "F.Cu" "B.Cu") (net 12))
 (via (at 132.4 106.8) (size 1.016) (drill 0.508) (layers "F.Cu" "B.Cu") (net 12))
 (segment (start 134.8 106.8) (end 137.271343 104.328657) (width 0.2) (layer "B.Cu") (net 12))
 (segment (start 137.271343 104.328657) (end 139.071343 104.328657) (width 0.2) (layer "B.Cu") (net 12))
 (segment (start 132.4 106.8) (end 134.8 106.8) (width 0.2) (layer "B.Cu") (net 12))
 (segment (start 157 95.4) (end 159.6 92.8) (width 0.2) (layer "F.Cu") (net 3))
 (segment (start 159.6 92.8) (end 164.4 92.8) (width 0.2) (layer "F.Cu") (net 3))
 (segment (start 154.6 95.4) (end 157 95.4) (width 0.2) (layer "F.Cu") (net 3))
 (segment (start 113.97 85.01) (end 131.81 85.01) (width 0.2) (layer "F.Cu") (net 10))
 (segment (start 146.2 114.4) (end 149.18 114.4) (width 0.2) (layer "F.Cu") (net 10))
 (segment (start 137.2 105.4) (end 146.2 114.4) (width 0.2) (layer "F.Cu") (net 10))
 (segment (start 137.2 90.4) (end 137.2 105.4) (width 0.2) (layer "F.Cu") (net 10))
 (segment (start 131.81 85.01) (end 137.2 90.4) (width 0.2) (layer "F.Cu") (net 10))
 (segment (start 135.8 105.8) (end 146.94 116.94) (width 0.2) (layer "F.Cu") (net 9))
 (segment (start 111.316865 77.39) (end 110 78.706865) (width 0.2) (layer "F.Cu") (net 9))
 (segment (start 133.6 94.4) (end 135.8 96.6) (width 0.2) (layer "F.Cu") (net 9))
 (segment (start 110 78.706865) (end 110 92.4) (width 0.2) (layer "F.Cu") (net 9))
 (segment (start 146.94 116.94) (end 149.18 116.94) (width 0.2) (layer "F.Cu") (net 9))
 (segment (start 113.69 77.39) (end 111.316865 77.39) (width 0.2) (layer "F.Cu") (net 9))
 (segment (start 112 94.4) (end 133.6 94.4) (width 0.2) (layer "F.Cu") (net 9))
 (segment (start 135.8 96.6) (end 135.8 105.8) (width 0.2) (layer "F.Cu") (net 9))
 (segment (start 110 92.4) (end 112 94.4) (width 0.2) (layer "F.Cu") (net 9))
 (segment (start 149.18 122.02) (end 146.82 122.02) (width 0.2) (layer "F.Cu") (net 7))
 (segment (start 146.82 122.02) (end 144.4 119.6) (width 0.2) (layer "F.Cu") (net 7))
 (segment (start 144.4 119.6) (end 144.4 117) (width 0.2) (layer "F.Cu") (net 7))
 (segment (start 145.1 101.7) (end 145.1 105.2) (width 0.2) (layer "F.Cu") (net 7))
 (segment (start 136.83 85.01) (end 136.83 85.29) (width 0.2) (layer "F.Cu") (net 7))
 (segment (start 136.83 85.29) (end 139.4 87.86) (width 0.2) (layer "F.Cu") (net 7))
 (segment (start 139.4 96) (end 145.1 101.7) (width 0.2) (layer "F.Cu") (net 7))
 (segment (start 139.4 87.86) (end 139.4 96) (width 0.2) (layer "F.Cu") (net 7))
 (via (at 144.4 117) (size 1.016) (drill 0.508) (layers "F.Cu" "B.Cu") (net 7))
 (via (at 145.1 105.2) (size 1.016) (drill 0.508) (layers "F.Cu" "B.Cu") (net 7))
 (segment (start 143.8 106.5) (end 143.8 116.4) (width 0.2) (layer "B.Cu") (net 7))
 (segment (start 143.8 116.4) (end 144.4 117) (width 0.2) (layer "B.Cu") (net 7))
 (segment (start 145.1 105.2) (end 143.8 106.5) (width 0.2) (layer "B.Cu") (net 7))
 (segment (start 130.2 95.8) (end 131.6 97.2) (width 0.2) (layer "F.Cu") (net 1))
 (segment (start 103 94.2) (end 104.6 95.8) (width 0.2) (layer "F.Cu") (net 1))
 (segment (start 104.6 95.8) (end 130.2 95.8) (width 0.2) (layer "F.Cu") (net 1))
 (segment (start 156.2 102.2) (end 156.2 105.6) (width 0.2) (layer "F.Cu") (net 1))
 (segment (start 156.2 105.6) (end 162.46 111.86) (width 0.2) (layer "F.Cu") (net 1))
 (segment (start 162.46 111.86) (end 164.42 111.86) (width 0.2) (layer "F.Cu") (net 1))
 (segment (start 102.6 90.2) (end 103 89.8) (width 0.2) (layer "F.Cu") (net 1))
 (segment (start 103 89.8) (end 103 94.2) (width 0.2) (layer "F.Cu") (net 1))
 (segment (start 155.4 101.4) (end 156.2 102.2) (width 0.2) (layer "F.Cu") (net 1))
 (via (at 131.6 97.2) (size 1.016) (drill 0.508) (layers "F.Cu" "B.Cu") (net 1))
 (via (at 155.4 101.4) (size 1.016) (drill 0.508) (layers "F.Cu" "B.Cu") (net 1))
 (segment (start 135 101.4) (end 133 99.4) (width 0.2) (layer "B.Cu") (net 1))
 (segment (start 133 99.4) (end 133 97.6) (width 0.2) (layer "B.Cu") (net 1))
 (segment (start 155.4 101.4) (end 135 101.4) (width 0.2) (layer "B.Cu") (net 1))
 (segment (start 132.6 97.2) (end 131.6 97.2) (width 0.2) (layer "B.Cu") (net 1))
 (segment (start 133 97.6) (end 132.6 97.2) (width 0.2) (layer "B.Cu") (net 1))
 (segment (start 100.5 116.3) (end 109.2 125) (width 0.2) (layer "F.Cu") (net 15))
 (segment (start 109.2 125) (end 161 125) (width 0.2) (layer "F.Cu") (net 15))
 (segment (start 162 121.9) (end 164.42 119.48) (width 0.2) (layer "F.Cu") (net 15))
 (segment (start 162 124) (end 162 121.9) (width 0.2) (layer "F.Cu") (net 15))
 (segment (start 86.05 116.2) (end 97.55 116.2) (width 0.2) (layer "F.Cu") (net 15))
 (segment (start 85.15 117.1) (end 86.05 116.2) (width 0.2) (layer "F.Cu") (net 15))
 (segment (start 97.55 116.2) (end 97.65 116.3) (width 0.2) (layer "F.Cu") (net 15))
 (segment (start 161 125) (end 162 124) (width 0.2) (layer "F.Cu") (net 15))
 (segment (start 97.65 116.3) (end 100.5 116.3) (width 0.2) (layer "F.Cu") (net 15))
 (segment (start 85.25 111.2) (end 97.55 111.2) (width 0.2) (layer "F.Cu") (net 17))
 (segment (start 97.65 111.3) (end 100.9 111.3) (width 0.2) (layer "F.Cu") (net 17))
 (segment (start 100.9 111.3) (end 110.2 120.6) (width 0.2) (layer "F.Cu") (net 17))
 (segment (start 97.55 111.2) (end 97.65 111.3) (width 0.2) (layer "F.Cu") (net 17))
 (segment (start 164.42 114.4) (end 161.8 114.4) (width 0.2) (layer "F.Cu") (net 17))
 (segment (start 110.2 120.6) (end 131.4 120.6) (width 0.2) (layer "F.Cu") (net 17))
 (segment (start 85.15 111.3) (end 85.25 111.2) (width 0.2) (layer "F.Cu") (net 17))
 (segment (start 131.4 120.6) (end 137.4 114.6) (width 0.2) (layer "F.Cu") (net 17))
 (segment (start 97.75 111.2) (end 97.65 111.3) (width 0.2) (layer "F.Cu") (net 17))
 (segment (start 161.8 114.4) (end 152.6 105.2) (width 0.2) (layer "F.Cu") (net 17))
 (via (at 152.6 105.2) (size 1.016) (drill 0.508) (layers "F.Cu" "B.Cu") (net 17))
 (via (at 137.4 114.6) (size 1.016) (drill 0.508) (layers "F.Cu" "B.Cu") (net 17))
 (segment (start 151 103.6) (end 143.6 103.6) (width 0.2) (layer "B.Cu") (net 17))
 (segment (start 137.5 114.6) (end 137.4 114.6) (width 0.2) (layer "B.Cu") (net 17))
 (segment (start 142.8 104.4) (end 142.8 109.3) (width 0.2) (layer "B.Cu") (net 17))
 (segment (start 152.6 105.2) (end 151 103.6) (width 0.2) (layer "B.Cu") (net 17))
 (segment (start 142.8 109.3) (end 137.5 114.6) (width 0.2) (layer "B.Cu") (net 17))
 (segment (start 143.6 103.6) (end 142.8 104.4) (width 0.2) (layer "B.Cu") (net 17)))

